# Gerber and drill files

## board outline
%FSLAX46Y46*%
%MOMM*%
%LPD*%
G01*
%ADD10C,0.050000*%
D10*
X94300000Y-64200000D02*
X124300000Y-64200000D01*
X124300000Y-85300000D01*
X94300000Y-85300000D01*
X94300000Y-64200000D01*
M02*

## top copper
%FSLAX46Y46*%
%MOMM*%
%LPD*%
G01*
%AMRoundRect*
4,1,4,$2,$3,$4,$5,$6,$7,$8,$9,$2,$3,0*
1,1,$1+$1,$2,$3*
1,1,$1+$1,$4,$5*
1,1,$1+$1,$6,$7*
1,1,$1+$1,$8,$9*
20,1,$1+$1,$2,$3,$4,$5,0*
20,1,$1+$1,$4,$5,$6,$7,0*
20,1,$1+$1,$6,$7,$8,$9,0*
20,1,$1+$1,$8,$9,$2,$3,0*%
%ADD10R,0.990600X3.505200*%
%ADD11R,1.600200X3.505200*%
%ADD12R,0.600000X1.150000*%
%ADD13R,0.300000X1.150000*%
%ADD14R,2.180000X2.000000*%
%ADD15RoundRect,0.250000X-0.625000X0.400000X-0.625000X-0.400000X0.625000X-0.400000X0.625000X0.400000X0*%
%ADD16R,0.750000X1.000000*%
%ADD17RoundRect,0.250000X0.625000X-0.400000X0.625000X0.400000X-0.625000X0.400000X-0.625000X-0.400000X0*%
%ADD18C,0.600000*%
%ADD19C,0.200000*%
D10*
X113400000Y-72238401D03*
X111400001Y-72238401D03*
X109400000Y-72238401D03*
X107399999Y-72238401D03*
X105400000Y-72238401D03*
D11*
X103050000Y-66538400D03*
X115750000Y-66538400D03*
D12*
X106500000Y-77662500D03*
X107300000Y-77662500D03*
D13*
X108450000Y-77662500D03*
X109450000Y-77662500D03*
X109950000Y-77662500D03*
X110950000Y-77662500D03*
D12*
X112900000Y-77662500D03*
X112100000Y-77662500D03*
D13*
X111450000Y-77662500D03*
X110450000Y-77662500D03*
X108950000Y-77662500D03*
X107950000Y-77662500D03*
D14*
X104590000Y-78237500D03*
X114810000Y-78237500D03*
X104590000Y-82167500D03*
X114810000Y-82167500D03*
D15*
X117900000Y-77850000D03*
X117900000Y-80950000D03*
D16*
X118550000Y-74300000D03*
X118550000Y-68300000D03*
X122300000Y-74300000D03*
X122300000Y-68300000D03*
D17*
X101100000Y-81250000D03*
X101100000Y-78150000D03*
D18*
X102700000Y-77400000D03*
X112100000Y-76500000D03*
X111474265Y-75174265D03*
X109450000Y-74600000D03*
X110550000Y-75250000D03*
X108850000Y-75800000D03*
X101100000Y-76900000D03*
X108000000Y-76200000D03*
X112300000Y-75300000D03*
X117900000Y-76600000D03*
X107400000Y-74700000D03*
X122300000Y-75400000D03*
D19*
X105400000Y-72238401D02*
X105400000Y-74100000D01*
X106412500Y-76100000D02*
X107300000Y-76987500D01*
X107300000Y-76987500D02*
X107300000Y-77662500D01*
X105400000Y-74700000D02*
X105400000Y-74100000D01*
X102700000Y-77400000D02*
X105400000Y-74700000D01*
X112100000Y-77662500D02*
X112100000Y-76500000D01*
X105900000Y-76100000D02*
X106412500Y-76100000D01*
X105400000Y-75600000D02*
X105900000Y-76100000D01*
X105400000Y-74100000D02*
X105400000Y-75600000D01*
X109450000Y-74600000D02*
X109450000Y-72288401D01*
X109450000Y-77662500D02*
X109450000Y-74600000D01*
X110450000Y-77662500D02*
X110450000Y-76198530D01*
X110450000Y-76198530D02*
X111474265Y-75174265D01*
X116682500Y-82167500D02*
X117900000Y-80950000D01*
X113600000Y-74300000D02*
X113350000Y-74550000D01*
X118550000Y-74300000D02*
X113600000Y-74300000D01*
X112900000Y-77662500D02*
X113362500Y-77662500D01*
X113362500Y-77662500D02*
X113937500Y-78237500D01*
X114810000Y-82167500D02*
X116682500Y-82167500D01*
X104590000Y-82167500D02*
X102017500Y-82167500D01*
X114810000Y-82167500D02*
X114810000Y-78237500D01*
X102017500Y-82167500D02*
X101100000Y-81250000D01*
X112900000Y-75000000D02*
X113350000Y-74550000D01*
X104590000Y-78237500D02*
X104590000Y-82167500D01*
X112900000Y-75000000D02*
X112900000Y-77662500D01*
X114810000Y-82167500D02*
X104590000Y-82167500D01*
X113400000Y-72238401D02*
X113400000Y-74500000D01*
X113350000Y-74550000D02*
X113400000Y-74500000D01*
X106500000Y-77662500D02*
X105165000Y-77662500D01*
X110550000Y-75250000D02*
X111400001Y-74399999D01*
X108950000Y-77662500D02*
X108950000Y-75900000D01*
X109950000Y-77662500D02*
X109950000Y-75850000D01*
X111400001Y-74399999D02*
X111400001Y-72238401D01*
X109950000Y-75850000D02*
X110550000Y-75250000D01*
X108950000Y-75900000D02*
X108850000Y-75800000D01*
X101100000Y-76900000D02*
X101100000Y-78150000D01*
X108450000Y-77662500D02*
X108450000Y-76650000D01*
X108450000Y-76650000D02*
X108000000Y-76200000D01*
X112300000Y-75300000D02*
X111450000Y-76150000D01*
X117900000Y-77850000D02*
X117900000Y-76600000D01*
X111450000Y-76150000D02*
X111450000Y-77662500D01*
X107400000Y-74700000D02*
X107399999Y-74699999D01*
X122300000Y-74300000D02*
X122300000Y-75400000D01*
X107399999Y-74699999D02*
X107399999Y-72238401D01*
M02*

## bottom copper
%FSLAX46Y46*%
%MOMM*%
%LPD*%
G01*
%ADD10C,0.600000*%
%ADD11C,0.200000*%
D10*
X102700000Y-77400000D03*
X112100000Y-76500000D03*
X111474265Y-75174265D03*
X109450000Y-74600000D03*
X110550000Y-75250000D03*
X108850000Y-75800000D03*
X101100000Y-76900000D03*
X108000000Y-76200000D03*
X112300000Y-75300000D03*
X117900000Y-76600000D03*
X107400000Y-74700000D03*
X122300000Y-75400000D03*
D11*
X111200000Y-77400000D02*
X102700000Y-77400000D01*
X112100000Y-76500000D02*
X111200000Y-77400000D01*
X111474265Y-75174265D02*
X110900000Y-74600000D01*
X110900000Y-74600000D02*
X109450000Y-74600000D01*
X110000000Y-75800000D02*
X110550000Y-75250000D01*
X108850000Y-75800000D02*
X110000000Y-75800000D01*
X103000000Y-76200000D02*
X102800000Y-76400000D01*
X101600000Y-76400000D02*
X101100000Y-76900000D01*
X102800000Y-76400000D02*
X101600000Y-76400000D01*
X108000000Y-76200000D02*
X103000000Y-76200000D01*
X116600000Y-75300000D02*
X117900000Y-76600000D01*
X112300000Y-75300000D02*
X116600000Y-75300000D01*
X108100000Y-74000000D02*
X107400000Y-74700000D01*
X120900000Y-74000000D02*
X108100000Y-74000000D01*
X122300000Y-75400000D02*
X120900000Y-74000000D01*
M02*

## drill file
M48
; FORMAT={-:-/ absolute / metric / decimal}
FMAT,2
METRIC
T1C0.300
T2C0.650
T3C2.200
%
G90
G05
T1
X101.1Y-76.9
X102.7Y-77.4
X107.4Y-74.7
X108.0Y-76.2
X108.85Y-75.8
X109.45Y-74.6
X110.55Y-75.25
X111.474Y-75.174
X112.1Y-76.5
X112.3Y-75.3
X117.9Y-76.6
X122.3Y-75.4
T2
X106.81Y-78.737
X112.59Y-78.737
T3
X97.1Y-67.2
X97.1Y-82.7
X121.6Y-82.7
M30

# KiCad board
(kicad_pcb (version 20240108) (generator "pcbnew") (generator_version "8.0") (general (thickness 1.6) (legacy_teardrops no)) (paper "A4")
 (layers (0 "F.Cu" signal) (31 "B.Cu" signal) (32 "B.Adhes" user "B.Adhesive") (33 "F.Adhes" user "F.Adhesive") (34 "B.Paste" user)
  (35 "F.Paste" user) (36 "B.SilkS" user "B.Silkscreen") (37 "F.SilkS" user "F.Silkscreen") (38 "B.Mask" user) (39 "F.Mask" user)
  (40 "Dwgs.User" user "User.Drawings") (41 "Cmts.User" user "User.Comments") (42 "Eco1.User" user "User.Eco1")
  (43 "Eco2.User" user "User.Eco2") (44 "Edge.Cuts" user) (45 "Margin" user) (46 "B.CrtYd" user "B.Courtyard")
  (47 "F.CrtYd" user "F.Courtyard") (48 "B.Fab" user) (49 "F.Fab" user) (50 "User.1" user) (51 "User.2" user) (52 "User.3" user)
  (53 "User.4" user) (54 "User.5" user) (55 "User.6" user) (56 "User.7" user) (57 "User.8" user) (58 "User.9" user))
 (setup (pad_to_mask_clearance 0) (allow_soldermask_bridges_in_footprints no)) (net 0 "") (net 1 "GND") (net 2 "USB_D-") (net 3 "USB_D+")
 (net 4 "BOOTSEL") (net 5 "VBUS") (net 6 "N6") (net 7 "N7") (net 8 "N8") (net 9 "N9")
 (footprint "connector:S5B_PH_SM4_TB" (layer "F.Cu") (at 109.4 68.782701)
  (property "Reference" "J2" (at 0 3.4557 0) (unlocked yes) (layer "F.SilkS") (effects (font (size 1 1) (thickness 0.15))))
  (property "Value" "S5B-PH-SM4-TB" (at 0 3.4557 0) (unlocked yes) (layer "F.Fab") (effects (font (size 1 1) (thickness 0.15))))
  (pad "1" smd rect (at 4 3.4557) (size 0.9906 3.5052) (layers "F.Cu" "F.Paste" "F.Mask") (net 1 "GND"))
  (pad "2" smd rect (at 2.000001 3.4557) (size 0.9906 3.5052) (layers "F.Cu" "F.Paste" "F.Mask") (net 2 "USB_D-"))
  (pad "3" smd rect (at 0 3.4557) (size 0.9906 3.5052) (layers "F.Cu" "F.Paste" "F.Mask") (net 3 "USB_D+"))
  (pad "4" smd rect (at -2.000001 3.4557) (size 0.9906 3.5052) (layers "F.Cu" "F.Paste" "F.Mask") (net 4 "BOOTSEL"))
  (pad "5" smd rect (at -4 3.4557) (size 0.9906 3.5052) (layers "F.Cu" "F.Paste" "F.Mask") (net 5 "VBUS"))
  (pad "6" smd rect (at -6.35 -2.244301) (size 1.6002 3.5052) (layers "F.Cu" "F.Paste" "F.Mask"))
  (pad "7" smd rect (at 6.35 -2.244301) (size 1.6002 3.5052) (layers "F.Cu" "F.Paste" "F.Mask")))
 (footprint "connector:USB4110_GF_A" (layer "F.Cu") (at 109.7 78.7375)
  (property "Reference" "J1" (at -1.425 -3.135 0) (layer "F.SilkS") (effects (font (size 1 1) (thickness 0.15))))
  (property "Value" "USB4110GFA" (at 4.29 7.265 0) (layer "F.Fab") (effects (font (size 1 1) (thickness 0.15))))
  (pad "" np_thru_hole circle (at -2.89 0) (size 0.65 0.65) (drill 0.65) (layers "*.Cu" "*.Mask"))
  (pad "" np_thru_hole circle (at 2.89 0) (size 0.65 0.65) (drill 0.65) (layers "*.Cu" "*.Mask"))
  (pad "A1/B12" smd rect (at -3.2 -1.075) (size 0.6 1.15) (layers "F.Cu" "F.Paste" "F.Mask") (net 1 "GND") (solder_mask_margin 0.102))
  (pad "A4/B9" smd rect (at -2.4 -1.075) (size 0.6 1.15) (layers "F.Cu" "F.Paste" "F.Mask") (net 5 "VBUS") (solder_mask_margin 0.102))
  (pad "A5" smd rect (at -1.25 -1.075) (size 0.3 1.15) (layers "F.Cu" "F.Paste" "F.Mask") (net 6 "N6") (solder_mask_margin 0.102))
  (pad "A6" smd rect (at -0.25 -1.075) (size 0.3 1.15) (layers "F.Cu" "F.Paste" "F.Mask") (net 3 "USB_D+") (solder_mask_margin 0.102))
  (pad "A7" smd rect (at 0.25 -1.075) (size 0.3 1.15) (layers "F.Cu" "F.Paste" "F.Mask") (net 2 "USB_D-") (solder_mask_margin 0.102))
  (pad "A8" smd rect (at 1.25 -1.075) (size 0.3 1.15) (layers "F.Cu" "F.Paste" "F.Mask") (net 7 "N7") (solder_mask_margin 0.102))
  (pad "B1/A12" smd rect (at 3.2 -1.075) (size 0.6 1.15) (layers "F.Cu" "F.Paste" "F.Mask") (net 1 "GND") (solder_mask_margin 0.102))
  (pad "B4/A9" smd rect (at 2.4 -1.075) (size 0.6 1.15) (layers "F.Cu" "F.Paste" "F.Mask") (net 5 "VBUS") (solder_mask_margin 0.102))
  (pad "B5" smd rect (at 1.75 -1.075) (size 0.3 1.15) (layers "F.Cu" "F.Paste" "F.Mask") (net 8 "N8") (solder_mask_margin 0.102))
  (pad "B6" smd rect (at 0.75 -1.075) (size 0.3 1.15) (layers "F.Cu" "F.Paste" "F.Mask") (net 3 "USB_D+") (solder_mask_margin 0.102))
  (pad "B7" smd rect (at -0.75 -1.075) (size 0.3 1.15) (layers "F.Cu" "F.Paste" "F.Mask") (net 2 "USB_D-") (solder_mask_margin 0.102))
  (pad "B8" smd rect (at -1.75 -1.075) (size 0.3 1.15) (layers "F.Cu" "F.Paste" "F.Mask") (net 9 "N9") (solder_mask_margin 0.102))
  (pad "S1" smd rect (at -5.11 -0.5) (size 2.18 2) (layers "F.Cu" "F.Paste" "F.Mask") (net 1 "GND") (solder_mask_margin 0.102))
  (pad "S2" smd rect (at 5.11 -0.5) (size 2.18 2) (layers "F.Cu" "F.Paste" "F.Mask") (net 1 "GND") (solder_mask_margin 0.102))
  (pad "S3" smd rect (at -5.11 3.43) (size 2.18 2) (layers "F.Cu" "F.Paste" "F.Mask") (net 1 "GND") (solder_mask_margin 0.102))
  (pad "S4" smd rect (at 5.11 3.43) (size 2.18 2) (layers "F.Cu" "F.Paste" "F.Mask") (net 1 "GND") (solder_mask_margin 0.102)))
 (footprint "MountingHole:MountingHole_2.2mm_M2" (layer "F.Cu") (at 121.6 82.7)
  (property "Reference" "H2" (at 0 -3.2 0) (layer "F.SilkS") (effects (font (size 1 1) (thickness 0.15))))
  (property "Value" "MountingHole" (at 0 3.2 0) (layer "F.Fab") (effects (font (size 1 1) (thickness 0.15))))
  (pad "" np_thru_hole circle (at 0 0) (size 2.2 2.2) (drill 2.2) (layers "*.Cu" "*.Mask")))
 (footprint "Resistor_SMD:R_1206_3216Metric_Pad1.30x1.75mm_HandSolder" (layer "F.Cu") (at 117.9 79.4 -90)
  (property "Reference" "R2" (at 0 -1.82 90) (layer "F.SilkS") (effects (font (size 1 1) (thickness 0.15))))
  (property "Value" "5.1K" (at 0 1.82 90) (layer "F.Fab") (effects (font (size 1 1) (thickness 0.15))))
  (pad "1" smd roundrect (at -1.55 0 270) (size 1.3 1.75) (layers "F.Cu" "F.Paste" "F.Mask") (roundrect_rratio 0.192308) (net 8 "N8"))
  (pad "2" smd roundrect (at 1.55 0 270) (size 1.3 1.75) (layers "F.Cu" "F.Paste" "F.Mask") (roundrect_rratio 0.192308) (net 1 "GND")))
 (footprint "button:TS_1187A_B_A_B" (layer "F.Cu") (at 120.425 71.3 90)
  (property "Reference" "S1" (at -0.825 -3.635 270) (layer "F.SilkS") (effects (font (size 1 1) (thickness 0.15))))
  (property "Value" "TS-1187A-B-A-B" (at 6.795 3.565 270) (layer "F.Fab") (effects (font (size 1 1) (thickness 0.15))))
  (pad "A" smd rect (at -3 -1.875 90) (size 1 0.75) (layers "F.Cu" "F.Paste" "F.Mask") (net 1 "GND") (solder_mask_margin 0.102))
  (pad "B" smd rect (at 3 -1.875 90) (size 1 0.75) (layers "F.Cu" "F.Paste" "F.Mask") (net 1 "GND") (solder_mask_margin 0.102))
  (pad "C" smd rect (at -3 1.875 90) (size 1 0.75) (layers "F.Cu" "F.Paste" "F.Mask") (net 4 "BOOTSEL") (solder_mask_margin 0.102))
  (pad "D" smd rect (at 3 1.875 90) (size 1 0.75) (layers "F.Cu" "F.Paste" "F.Mask") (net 4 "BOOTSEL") (solder_mask_margin 0.102)))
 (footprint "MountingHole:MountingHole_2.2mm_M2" (layer "F.Cu") (at 97.1 67.2)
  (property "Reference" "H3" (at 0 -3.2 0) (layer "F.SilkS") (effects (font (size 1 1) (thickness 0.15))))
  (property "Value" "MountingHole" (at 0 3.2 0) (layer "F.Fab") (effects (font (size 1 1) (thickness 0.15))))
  (pad "" np_thru_hole circle (at 0 0) (size 2.2 2.2) (drill 2.2) (layers "*.Cu" "*.Mask")))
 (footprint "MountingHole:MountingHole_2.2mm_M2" (layer "F.Cu") (at 97.1 82.7)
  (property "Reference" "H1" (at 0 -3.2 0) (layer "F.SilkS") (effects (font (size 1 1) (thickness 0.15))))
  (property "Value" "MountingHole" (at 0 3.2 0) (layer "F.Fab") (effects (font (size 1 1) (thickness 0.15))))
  (pad "" np_thru_hole circle (at 0 0) (size 2.2 2.2) (drill 2.2) (layers "*.Cu" "*.Mask")))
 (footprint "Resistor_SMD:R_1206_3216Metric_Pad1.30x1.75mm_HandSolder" (layer "F.Cu") (at 101.1 79.7 90)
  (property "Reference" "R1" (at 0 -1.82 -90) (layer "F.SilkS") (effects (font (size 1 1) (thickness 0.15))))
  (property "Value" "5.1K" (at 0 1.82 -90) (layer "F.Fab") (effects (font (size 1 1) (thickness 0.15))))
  (pad "1" smd roundrect (at -1.55 0 90) (size 1.3 1.75) (layers "F.Cu" "F.Paste" "F.Mask") (roundrect_rratio 0.192308) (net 1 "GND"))
  (pad "2" smd roundrect (at 1.55 0 90) (size 1.3 1.75) (layers "F.Cu" "F.Paste" "F.Mask") (roundrect_rratio 0.192308) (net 6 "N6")))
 (gr_rect (start 94.3 64.2) (end 124.3 85.3) (stroke (width 0.05) (type default)) (fill none) (layer "Edge.Cuts"))
 (segment (start 105.4 72.238401) (end 105.4 74.1) (width 0.2) (layer "F.Cu") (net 5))
 (segment (start 106.4125 76.1) (end 107.3 76.9875) (width 0.2) (layer "F.Cu") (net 5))
 (segment (start 107.3 76.9875) (end 107.3 77.6625) (width 0.2) (layer "F.Cu") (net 5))
 (segment (start 105.4 74.7) (end 105.4 74.1) (width 0.2) (layer "F.Cu") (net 5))
 (segment (start 102.7 77.4) (end 105.4 74.7) (width 0.2) (layer "F.Cu") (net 5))
 (segment (start 112.1 77.6625) (end 112.1 76.5) (width 0.2) (layer "F.Cu") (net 5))
 (segment (start 105.9 76.1) (end 106.4125 76.1) (width 0.2) (layer "F.Cu") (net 5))
 (segment (start 105.4 75.6) (end 105.9 76.1) (width 0.2) (layer "F.Cu") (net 5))
 (segment (start 105.4 74.1) (end 105.4 75.6) (width 0.2) (layer "F.Cu") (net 5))
 (via (at 102.7 77.4) (size 0.6) (drill 0.3) (layers "F.Cu" "B.Cu") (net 5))
 (via (at 112.1 76.5) (size 0.6) (drill 0.3) (layers "F.Cu" "B.Cu") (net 5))
 (segment (start 111.2 77.4) (end 102.7 77.4) (width 0.2) (layer "B.Cu") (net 5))
 (segment (start 112.1 76.5) (end 111.2 77.4) (width 0.2) (layer "B.Cu") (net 5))
 (segment (start 109.45 74.6) (end 109.45 72.288401) (width 0.2) (layer "F.Cu") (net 3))
 (segment (start 109.45 77.6625) (end 109.45 74.6) (width 0.2) (layer "F.Cu") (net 3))
 (segment (start 110.45 77.6625) (end 110.45 76.19853) (width 0.2) (layer "F.Cu") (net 3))
 (segment (start 110.45 76.19853) (end 111.474265 75.174265) (width 0.2) (layer "F.Cu") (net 3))
 (via (at 111.474265 75.174265) (size 0.6) (drill 0.3) (layers "F.Cu" "B.Cu") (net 3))
 (via (at 109.45 74.6) (size 0.6) (drill 0.3) (layers "F.Cu" "B.Cu") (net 3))
 (segment (start 111.474265 75.174265) (end 110.9 74.6) (width 0.2) (layer "B.Cu") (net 3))
 (segment (start 110.9 74.6) (end 109.45 74.6) (width 0.2) (layer "B.Cu") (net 3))
 (segment (start 116.6825 82.1675) (end 117.9 80.95) (width 0.2) (layer "F.Cu") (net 1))
 (segment (start 113.6 74.3) (end 113.35 74.55) (width 0.2) (layer "F.Cu") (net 1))
 (segment (start 118.55 74.3) (end 113.6 74.3) (width 0.2) (layer "F.Cu") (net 1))
 (segment (start 112.9 77.6625) (end 113.3625 77.6625) (width 0.2) (layer "F.Cu") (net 1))
 (segment (start 113.3625 77.6625) (end 113.9375 78.2375) (width 0.2) (layer "F.Cu") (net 1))
 (segment (start 114.81 82.1675) (end 116.6825 82.1675) (width 0.2) (layer "F.Cu") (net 1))
 (segment (start 104.59 82.1675) (end 102.0175 82.1675) (width 0.2) (layer "F.Cu") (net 1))
 (segment (start 114.81 82.1675) (end 114.81 78.2375) (width 0.2) (layer "F.Cu") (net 1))
 (segment (start 102.0175 82.1675) (end 101.1 81.25) (width 0.2) (layer "F.Cu") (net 1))
 (segment (start 112.9 75) (end 113.35 74.55) (width 0.2) (layer "F.Cu") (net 1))
 (segment (start 104.59 78.2375) (end 104.59 82.1675) (width 0.2) (layer "F.Cu") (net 1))
 (segment (start 112.9 75) (end 112.9 77.6625) (width 0.2) (layer "F.Cu") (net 1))
 (segment (start 114.81 82.1675) (end 104.59 82.1675) (width 0.2) (layer "F.Cu") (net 1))
 (segment (start 113.4 72.238401) (end 113.4 74.5) (width 0.2) (layer "F.Cu") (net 1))
 (segment (start 113.35 74.55) (end 113.4 74.5) (width 0.2) (layer "F.Cu") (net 1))
 (segment (start 106.5 77.6625) (end 105.165 77.6625) (width 0.2) (layer "F.Cu") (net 1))
 (segment (start 110.55 75.25) (end 111.400001 74.399999) (width 0.2) (layer "F.Cu") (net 2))
 (segment (start 108.95 77.6625) (end 108.95 75.9) (width 0.2) (layer "F.Cu") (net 2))
 (segment (start 109.95 77.6625) (end 109.95 75.85) (width 0.2) (layer "F.Cu") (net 2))
 (segment (start 111.400001 74.399999) (end 111.400001 72.238401) (width 0.2) (layer "F.Cu") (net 2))
 (segment (start 109.95 75.85) (end 110.55 75.25) (width 0.2) (layer "F.Cu") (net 2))
 (segment (start 108.95 75.9) (end 108.85 75.8) (width 0.2) (layer "F.Cu") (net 2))
 (via (at 110.55 75.25) (size 0.6) (drill 0.3) (layers "F.Cu" "B.Cu") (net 2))
 (via (at 108.85 75.8) (size 0.6) (drill 0.3) (layers "F.Cu" "B.Cu") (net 2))
 (segment (start 110 75.8) (end 110.55 75.25) (width 0.2) (layer "B.Cu") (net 2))
 (segment (start 108.85 75.8) (end 110 75.8) (width 0.2) (layer "B.Cu") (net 2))
 (segment (start 101.1 76.9) (end 101.1 78.15) (width 0.2) (layer "F.Cu") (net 6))
 (segment (start 108.45 77.6625) (end 108.45 76.65) (width 0.2) (layer "F.Cu") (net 6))
 (segment (start 108.45 76.65) (end 108 76.2) (width 0.2) (layer "F.Cu") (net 6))
 (via (at 101.1 76.9) (size 0.6) (drill 0.3) (layers "F.Cu" "B.Cu") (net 6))
 (via (at 108 76.2) (size 0.6) (drill 0.3) (layers "F.Cu" "B.Cu") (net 6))
 (segment (start 103 76.2) (end 102.8 76.4) (width 0.2) (layer "B.Cu") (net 6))
 (segment (start 101.6 76.4) (end 101.1 76.9) (width 0.2) (layer "B.Cu") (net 6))
 (segment (start 102.8 76.4) (end 101.6 76.4) (width 0.2) (layer "B.Cu") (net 6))
 (segment (start 108 76.2) (end 103 76.2) (width 0.2) (layer "B.Cu") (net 6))
 (segment (start 112.3 75.3) (end 111.45 76.15) (width 0.2) (layer "F.Cu") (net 8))
 (segment (start 117.9 77.85) (end 117.9 76.6) (width 0.2) (layer "F.Cu") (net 8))
 (segment (start 111.45 76.15) (end 111.45 77.6625) (width 0.2) (layer "F.Cu") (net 8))
 (via (at 112.3 75.3) (size 0.6) (drill 0.3) (layers "F.Cu" "B.Cu") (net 8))
 (via (at 117.9 76.6) (size 0.6) (drill 0.3) (layers "F.Cu" "B.Cu") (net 8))
 (segment (start 116.6 75.3) (end 117.9 76.6) (width 0.2) (layer "B.Cu") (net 8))
 (segment (start 112.3 75.3) (end 116.6 75.3) (width 0.2) (layer "B.Cu") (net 8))
 (segment (start 107.4 74.7) (end 107.399999 74.699999) (width 0.2) (layer "F.Cu") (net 4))
 (segment (start 122.3 74.3) (end 122.3 75.4) (width 0.2) (layer "F.Cu") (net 4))
 (segment (start 107.399999 74.699999) (end 107.399999 72.238401) (width 0.2) (layer "F.Cu") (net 4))
 (via (at 107.4 74.7) (size 0.6) (drill 0.3) (layers "F.Cu" "B.Cu") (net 4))
 (via (at 122.3 75.4) (size 0.6) (drill 0.3) (layers "F.Cu" "B.Cu") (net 4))
 (segment (start 108.1 74) (end 107.4 74.7) (width 0.2) (layer "B.Cu") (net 4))
 (segment (start 120.9 74) (end 108.1 74) (width 0.2) (layer "B.Cu") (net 4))
 (segment (start 122.3 75.4) (end 120.9 74) (width 0.2) (layer "B.Cu") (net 4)))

